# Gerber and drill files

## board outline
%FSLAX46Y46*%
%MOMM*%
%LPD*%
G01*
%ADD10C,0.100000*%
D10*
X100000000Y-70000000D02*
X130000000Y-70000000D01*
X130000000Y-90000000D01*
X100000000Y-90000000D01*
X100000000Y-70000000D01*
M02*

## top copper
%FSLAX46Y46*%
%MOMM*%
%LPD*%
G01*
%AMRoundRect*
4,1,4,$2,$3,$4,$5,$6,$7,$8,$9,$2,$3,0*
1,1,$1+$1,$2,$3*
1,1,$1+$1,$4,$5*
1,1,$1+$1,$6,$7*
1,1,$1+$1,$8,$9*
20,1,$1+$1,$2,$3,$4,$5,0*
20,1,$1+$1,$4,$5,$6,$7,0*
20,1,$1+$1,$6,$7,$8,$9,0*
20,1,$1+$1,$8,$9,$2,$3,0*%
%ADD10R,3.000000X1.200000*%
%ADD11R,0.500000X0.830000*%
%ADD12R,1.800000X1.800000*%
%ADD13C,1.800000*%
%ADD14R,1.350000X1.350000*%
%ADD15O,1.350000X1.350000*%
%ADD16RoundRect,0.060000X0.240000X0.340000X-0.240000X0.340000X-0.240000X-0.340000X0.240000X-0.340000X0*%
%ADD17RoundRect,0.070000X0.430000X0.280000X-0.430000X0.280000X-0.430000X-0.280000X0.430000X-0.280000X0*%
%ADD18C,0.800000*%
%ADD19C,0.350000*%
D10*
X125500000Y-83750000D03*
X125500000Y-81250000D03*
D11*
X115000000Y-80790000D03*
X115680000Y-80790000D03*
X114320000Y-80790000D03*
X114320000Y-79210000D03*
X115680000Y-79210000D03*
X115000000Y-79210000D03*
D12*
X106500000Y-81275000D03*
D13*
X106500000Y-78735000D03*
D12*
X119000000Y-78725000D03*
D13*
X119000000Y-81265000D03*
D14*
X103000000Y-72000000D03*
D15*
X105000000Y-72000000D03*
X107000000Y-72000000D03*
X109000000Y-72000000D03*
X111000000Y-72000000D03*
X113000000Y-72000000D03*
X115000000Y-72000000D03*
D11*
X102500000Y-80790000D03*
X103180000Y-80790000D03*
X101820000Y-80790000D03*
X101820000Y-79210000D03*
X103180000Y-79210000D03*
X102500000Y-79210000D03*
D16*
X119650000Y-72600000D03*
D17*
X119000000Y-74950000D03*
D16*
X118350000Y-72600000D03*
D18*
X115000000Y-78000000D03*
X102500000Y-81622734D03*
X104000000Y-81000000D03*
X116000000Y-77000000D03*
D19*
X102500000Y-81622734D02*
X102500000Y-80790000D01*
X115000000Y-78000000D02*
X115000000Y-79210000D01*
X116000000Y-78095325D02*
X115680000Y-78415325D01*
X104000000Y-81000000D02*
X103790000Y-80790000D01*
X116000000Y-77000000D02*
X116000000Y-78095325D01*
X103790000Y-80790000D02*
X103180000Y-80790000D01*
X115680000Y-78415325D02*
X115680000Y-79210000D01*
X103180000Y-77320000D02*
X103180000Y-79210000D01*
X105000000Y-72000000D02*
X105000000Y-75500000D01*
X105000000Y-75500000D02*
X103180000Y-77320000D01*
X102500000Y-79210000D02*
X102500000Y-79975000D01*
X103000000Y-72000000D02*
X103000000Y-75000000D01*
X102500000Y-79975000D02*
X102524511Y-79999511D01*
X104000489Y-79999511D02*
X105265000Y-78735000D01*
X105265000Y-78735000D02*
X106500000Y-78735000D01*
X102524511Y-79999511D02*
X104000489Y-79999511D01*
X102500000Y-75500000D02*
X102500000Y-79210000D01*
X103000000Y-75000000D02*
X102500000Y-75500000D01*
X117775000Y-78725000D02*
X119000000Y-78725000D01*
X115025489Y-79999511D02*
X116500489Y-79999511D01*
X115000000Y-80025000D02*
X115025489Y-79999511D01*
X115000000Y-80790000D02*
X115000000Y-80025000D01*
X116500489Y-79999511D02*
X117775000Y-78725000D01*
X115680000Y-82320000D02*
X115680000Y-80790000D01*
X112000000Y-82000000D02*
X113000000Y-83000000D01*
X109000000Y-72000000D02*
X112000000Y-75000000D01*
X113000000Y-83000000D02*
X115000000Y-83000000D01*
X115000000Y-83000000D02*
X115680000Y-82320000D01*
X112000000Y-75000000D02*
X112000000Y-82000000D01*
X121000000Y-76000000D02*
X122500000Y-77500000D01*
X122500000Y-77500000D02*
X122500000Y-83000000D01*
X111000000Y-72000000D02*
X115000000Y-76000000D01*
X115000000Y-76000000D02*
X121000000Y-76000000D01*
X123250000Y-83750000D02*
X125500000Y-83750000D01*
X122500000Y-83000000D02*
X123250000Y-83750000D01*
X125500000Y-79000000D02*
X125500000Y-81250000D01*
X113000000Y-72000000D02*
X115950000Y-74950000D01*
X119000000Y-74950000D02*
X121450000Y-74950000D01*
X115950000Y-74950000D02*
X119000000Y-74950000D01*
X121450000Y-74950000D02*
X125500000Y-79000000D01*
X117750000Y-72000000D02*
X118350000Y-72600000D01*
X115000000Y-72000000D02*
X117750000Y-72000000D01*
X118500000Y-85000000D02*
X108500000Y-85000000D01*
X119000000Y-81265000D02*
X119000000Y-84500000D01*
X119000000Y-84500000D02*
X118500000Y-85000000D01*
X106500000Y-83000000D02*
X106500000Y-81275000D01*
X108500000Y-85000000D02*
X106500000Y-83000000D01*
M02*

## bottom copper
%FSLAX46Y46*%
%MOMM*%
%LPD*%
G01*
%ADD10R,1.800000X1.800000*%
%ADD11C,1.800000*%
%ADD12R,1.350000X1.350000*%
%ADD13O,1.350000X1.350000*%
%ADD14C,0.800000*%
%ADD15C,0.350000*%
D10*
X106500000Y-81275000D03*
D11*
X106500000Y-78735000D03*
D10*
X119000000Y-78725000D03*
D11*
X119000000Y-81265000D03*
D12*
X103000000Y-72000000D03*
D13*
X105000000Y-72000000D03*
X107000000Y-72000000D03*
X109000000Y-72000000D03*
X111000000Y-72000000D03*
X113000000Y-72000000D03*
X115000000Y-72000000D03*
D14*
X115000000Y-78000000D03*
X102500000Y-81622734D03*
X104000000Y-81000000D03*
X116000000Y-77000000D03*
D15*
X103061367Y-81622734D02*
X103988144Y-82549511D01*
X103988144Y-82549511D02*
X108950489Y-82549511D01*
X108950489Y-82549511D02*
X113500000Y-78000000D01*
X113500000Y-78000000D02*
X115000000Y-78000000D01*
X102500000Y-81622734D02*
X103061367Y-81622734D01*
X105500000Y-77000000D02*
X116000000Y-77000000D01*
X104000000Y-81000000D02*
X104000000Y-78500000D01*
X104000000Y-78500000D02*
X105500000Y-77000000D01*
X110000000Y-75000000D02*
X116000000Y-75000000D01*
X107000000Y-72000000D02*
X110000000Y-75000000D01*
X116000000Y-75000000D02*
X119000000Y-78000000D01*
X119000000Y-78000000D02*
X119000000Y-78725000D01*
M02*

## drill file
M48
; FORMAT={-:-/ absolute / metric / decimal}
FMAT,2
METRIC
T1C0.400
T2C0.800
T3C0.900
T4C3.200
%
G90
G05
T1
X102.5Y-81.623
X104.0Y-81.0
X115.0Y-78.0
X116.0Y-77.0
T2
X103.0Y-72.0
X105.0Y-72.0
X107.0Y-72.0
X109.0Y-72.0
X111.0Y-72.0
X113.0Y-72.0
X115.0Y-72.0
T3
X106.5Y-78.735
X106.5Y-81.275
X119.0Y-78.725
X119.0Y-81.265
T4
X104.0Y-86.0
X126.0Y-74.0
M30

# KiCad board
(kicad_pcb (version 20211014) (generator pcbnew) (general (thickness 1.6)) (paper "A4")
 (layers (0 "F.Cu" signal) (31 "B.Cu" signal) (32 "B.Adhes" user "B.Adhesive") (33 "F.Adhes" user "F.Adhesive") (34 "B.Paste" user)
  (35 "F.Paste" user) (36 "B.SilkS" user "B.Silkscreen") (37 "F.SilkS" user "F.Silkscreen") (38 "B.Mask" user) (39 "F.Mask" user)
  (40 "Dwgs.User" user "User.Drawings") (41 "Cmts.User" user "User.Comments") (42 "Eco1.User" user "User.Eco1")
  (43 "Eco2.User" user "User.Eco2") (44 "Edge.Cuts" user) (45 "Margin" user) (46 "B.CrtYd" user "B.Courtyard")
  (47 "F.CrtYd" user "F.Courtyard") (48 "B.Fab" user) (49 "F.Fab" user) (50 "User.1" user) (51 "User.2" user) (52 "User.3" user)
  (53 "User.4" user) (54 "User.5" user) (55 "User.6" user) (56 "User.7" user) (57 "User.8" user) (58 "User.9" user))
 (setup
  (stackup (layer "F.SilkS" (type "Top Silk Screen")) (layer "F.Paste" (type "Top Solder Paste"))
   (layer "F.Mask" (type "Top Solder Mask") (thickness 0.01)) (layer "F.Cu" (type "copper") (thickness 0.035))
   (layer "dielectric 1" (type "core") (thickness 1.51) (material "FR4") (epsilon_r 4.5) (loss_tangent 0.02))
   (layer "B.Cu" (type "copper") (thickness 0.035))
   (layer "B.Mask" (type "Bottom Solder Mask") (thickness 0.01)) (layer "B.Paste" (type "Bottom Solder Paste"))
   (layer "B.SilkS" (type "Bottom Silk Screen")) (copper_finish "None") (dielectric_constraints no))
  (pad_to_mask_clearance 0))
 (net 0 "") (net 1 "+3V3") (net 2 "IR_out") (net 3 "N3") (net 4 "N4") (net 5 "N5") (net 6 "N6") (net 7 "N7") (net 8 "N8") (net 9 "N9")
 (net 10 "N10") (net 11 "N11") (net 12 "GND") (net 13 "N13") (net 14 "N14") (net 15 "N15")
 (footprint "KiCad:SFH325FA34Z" (layer "F.Cu") (at 125.5 82.5 90)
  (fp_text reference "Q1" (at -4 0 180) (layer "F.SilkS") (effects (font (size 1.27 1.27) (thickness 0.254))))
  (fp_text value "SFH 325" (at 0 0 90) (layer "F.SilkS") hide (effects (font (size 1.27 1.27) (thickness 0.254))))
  (pad "1" smd rect (at -1.25 0 90) (size 1.2 3) (layers "F.Cu" "F.Paste" "F.Mask") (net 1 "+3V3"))
  (pad "2" smd rect (at 1.25 0 90) (size 1.2 3) (layers "F.Cu" "F.Paste" "F.Mask") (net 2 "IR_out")))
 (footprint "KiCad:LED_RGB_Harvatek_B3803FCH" (layer "F.Cu") (at 115 80 180)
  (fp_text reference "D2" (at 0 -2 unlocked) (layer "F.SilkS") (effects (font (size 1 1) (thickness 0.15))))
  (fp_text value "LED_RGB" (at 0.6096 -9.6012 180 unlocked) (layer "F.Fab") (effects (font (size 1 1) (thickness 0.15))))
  (pad "1" smd rect (at 0 -0.79 180) (size 0.5 0.83) (layers "F.Cu" "F.Paste" "F.Mask") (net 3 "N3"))
  (pad "2" smd rect (at -0.68 -0.79 180) (size 0.5 0.83) (layers "F.Cu" "F.Paste" "F.Mask") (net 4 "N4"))
  (pad "3" smd rect (at 0.68 -0.79 180) (size 0.5 0.83) (layers "F.Cu" "F.Paste" "F.Mask") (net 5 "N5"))
  (pad "4" smd rect (at 0.68 0.79 180) (size 0.5 0.83) (layers "F.Cu" "F.Paste" "F.Mask") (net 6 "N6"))
  (pad "5" smd rect (at -0.68 0.79 180) (size 0.5 0.83) (layers "F.Cu" "F.Paste" "F.Mask") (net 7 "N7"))
  (pad "6" smd rect (at 0 0.79 180) (size 0.5 0.83) (layers "F.Cu" "F.Paste" "F.Mask") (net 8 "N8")))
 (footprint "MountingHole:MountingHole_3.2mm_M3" (layer "F.Cu") (at 104 86)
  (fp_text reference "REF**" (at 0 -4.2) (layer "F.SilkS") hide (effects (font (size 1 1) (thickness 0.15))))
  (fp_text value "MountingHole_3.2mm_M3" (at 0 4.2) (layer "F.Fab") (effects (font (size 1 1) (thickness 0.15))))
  (pad "" np_thru_hole circle (at 0 0) (size 3.2 3.2) (drill 3.2) (layers *.Cu *.Mask)))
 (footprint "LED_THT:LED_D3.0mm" (layer "F.Cu") (at 106.5 81.275 90)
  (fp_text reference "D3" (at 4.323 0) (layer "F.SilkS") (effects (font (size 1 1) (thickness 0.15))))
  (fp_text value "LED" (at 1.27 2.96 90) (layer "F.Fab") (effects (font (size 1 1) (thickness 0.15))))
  (pad "1" thru_hole rect (at 0 0 90) (size 1.8 1.8) (drill 0.9) (layers *.Cu *.Mask) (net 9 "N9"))
  (pad "2" thru_hole circle (at 2.54 0 90) (size 1.8 1.8) (drill 0.9) (layers *.Cu *.Mask) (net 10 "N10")))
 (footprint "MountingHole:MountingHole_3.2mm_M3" (layer "F.Cu") (at 126 74)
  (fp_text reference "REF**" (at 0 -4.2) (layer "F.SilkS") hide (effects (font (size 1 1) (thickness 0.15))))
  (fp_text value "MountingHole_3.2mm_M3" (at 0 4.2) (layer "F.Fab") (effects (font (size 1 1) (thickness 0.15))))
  (pad "" np_thru_hole circle (at 0 0) (size 3.2 3.2) (drill 3.2) (layers *.Cu *.Mask)))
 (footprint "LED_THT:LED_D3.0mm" (layer "F.Cu") (at 119 78.725 -90)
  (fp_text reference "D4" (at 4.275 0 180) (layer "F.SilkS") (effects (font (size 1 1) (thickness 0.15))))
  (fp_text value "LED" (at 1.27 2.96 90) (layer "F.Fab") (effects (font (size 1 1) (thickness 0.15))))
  (pad "1" thru_hole rect (at 0 0 270) (size 1.8 1.8) (drill 0.9) (layers *.Cu *.Mask) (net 3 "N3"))
  (pad "2" thru_hole circle (at 2.54 0 270) (size 1.8 1.8) (drill 0.9) (layers *.Cu *.Mask) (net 9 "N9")))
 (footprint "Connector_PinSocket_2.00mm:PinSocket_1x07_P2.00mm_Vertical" (layer "F.Cu") (at 103 72 90)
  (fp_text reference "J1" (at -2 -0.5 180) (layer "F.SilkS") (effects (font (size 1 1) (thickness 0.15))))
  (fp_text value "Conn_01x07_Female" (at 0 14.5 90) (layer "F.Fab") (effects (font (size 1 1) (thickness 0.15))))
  (pad "1" thru_hole rect (at 0 0 90) (size 1.35 1.35) (drill 0.8) (layers *.Cu *.Mask) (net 10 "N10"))
  (pad "2" thru_hole oval (at 0 2 90) (size 1.35 1.35) (drill 0.8) (layers *.Cu *.Mask) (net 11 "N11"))
  (pad "3" thru_hole oval (at 0 4 90) (size 1.35 1.35) (drill 0.8) (layers *.Cu *.Mask) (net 3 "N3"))
  (pad "4" thru_hole oval (at 0 6 90) (size 1.35 1.35) (drill 0.8) (layers *.Cu *.Mask) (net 4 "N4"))
  (pad "5" thru_hole oval (at 0 8 90) (size 1.35 1.35) (drill 0.8) (layers *.Cu *.Mask) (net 1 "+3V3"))
  (pad "6" thru_hole oval (at 0 10 90) (size 1.35 1.35) (drill 0.8) (layers *.Cu *.Mask) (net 2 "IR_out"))
  (pad "7" thru_hole oval (at 0 12 90) (size 1.35 1.35) (drill 0.8) (layers *.Cu *.Mask) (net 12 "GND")))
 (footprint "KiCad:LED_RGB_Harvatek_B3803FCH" (layer "F.Cu") (at 102.5 80 180)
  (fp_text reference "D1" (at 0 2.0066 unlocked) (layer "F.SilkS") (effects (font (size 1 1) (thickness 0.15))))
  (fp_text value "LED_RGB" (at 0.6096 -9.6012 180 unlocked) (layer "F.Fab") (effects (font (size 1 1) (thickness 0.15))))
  (pad "1" smd rect (at 0 -0.79 180) (size 0.5 0.83) (layers "F.Cu" "F.Paste" "F.Mask") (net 8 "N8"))
  (pad "2" smd rect (at -0.68 -0.79 180) (size 0.5 0.83) (layers "F.Cu" "F.Paste" "F.Mask") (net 7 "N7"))
  (pad "3" smd rect (at 0.68 -0.79 180) (size 0.5 0.83) (layers "F.Cu" "F.Paste" "F.Mask") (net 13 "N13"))
  (pad "4" smd rect (at 0.68 0.79 180) (size 0.5 0.83) (layers "F.Cu" "F.Paste" "F.Mask") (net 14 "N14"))
  (pad "5" smd rect (at -0.68 0.79 180) (size 0.5 0.83) (layers "F.Cu" "F.Paste" "F.Mask") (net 11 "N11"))
  (pad "6" smd rect (at 0 0.79 180) (size 0.5 0.83) (layers "F.Cu" "F.Paste" "F.Mask") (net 10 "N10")))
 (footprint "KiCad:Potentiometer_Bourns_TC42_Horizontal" (layer "F.Cu") (at 119 74 180)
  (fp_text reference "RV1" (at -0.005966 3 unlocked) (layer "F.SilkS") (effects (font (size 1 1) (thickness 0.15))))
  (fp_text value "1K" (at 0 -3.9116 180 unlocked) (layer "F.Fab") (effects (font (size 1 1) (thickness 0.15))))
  (pad "1" smd roundrect (at -0.65 1.4 180) (size 0.6 0.8) (layers "F.Cu" "F.Paste" "F.Mask") (roundrect_rratio 0.1) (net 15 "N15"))
  (pad "2" smd roundrect (at 0 -0.95 180) (size 1 0.7) (layers "F.Cu" "F.Paste" "F.Mask") (roundrect_rratio 0.1) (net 2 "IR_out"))
  (pad "3" smd roundrect (at 0.65 1.4 180) (size 0.6 0.8) (layers "F.Cu" "F.Paste" "F.Mask") (roundrect_rratio 0.1) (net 12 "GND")))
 (gr_rect (start 100 70) (end 130 90) (layer "Edge.Cuts") (width 0.1) (fill none))
 (segment (start 102.5 81.622734) (end 102.5 80.79) (width 0.35) (layer "F.Cu") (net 8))
 (segment (start 115 78) (end 115 79.21) (width 0.35) (layer "F.Cu") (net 8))
 (via (at 115 78) (size 0.8) (drill 0.4) (layers "F.Cu" "B.Cu") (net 8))
 (via (at 102.5 81.622734) (size 0.8) (drill 0.4) (layers "F.Cu" "B.Cu") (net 8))
 (segment (start 103.061367 81.622734) (end 103.988144 82.549511) (width 0.35) (layer "B.Cu") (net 8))
 (segment (start 103.988144 82.549511) (end 108.950489 82.549511) (width 0.35) (layer "B.Cu") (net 8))
 (segment (start 108.950489 82.549511) (end 113.5 78) (width 0.35) (layer "B.Cu") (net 8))
 (segment (start 113.5 78) (end 115 78) (width 0.35) (layer "B.Cu") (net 8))
 (segment (start 102.5 81.622734) (end 103.061367 81.622734) (width 0.35) (layer "B.Cu") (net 8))
 (segment (start 116 78.095325) (end 115.68 78.415325) (width 0.35) (layer "F.Cu") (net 7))
 (segment (start 104 81) (end 103.79 80.79) (width 0.35) (layer "F.Cu") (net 7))
 (segment (start 116 77) (end 116 78.095325) (width 0.35) (layer "F.Cu") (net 7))
 (segment (start 103.79 80.79) (end 103.18 80.79) (width 0.35) (layer "F.Cu") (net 7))
 (segment (start 115.68 78.415325) (end 115.68 79.21) (width 0.35) (layer "F.Cu") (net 7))
 (via (at 104 81) (size 0.8) (drill 0.4) (layers "F.Cu" "B.Cu") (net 7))
 (via (at 116 77) (size 0.8) (drill 0.4) (layers "F.Cu" "B.Cu") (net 7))
 (segment (start 105.5 77) (end 116 77) (width 0.35) (layer "B.Cu") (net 7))
 (segment (start 104 81) (end 104 78.5) (width 0.35) (layer "B.Cu") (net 7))
 (segment (start 104 78.5) (end 105.5 77) (width 0.35) (layer "B.Cu") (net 7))
 (segment (start 103.18 77.32) (end 103.18 79.21) (width 0.35) (layer "F.Cu") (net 11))
 (segment (start 105 72) (end 105 75.5) (width 0.35) (layer "F.Cu") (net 11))
 (segment (start 105 75.5) (end 103.18 77.32) (width 0.35) (layer "F.Cu") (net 11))
 (segment (start 102.5 79.21) (end 102.5 79.975) (width 0.35) (layer "F.Cu") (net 10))
 (segment (start 103 72) (end 103 75) (width 0.35) (layer "F.Cu") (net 10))
 (segment (start 102.5 79.975) (end 102.524511 79.999511) (width 0.35) (layer "F.Cu") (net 10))
 (segment (start 104.000489 79.999511) (end 105.265 78.735) (width 0.35) (layer "F.Cu") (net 10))
 (segment (start 105.265 78.735) (end 106.5 78.735) (width 0.35) (layer "F.Cu") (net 10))
 (segment (start 102.524511 79.999511) (end 104.000489 79.999511) (width 0.35) (layer "F.Cu") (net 10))
 (segment (start 102.5 75.5) (end 102.5 79.21) (width 0.35) (layer "F.Cu") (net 10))
 (segment (start 103 75) (end 102.5 75.5) (width 0.35) (layer "F.Cu") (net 10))
 (segment (start 117.775 78.725) (end 119 78.725) (width 0.35) (layer "F.Cu") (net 3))
 (segment (start 115.025489 79.999511) (end 116.500489 79.999511) (width 0.35) (layer "F.Cu") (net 3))
 (segment (start 115 80.025) (end 115.025489 79.999511) (width 0.35) (layer "F.Cu") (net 3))
 (segment (start 115 80.79) (end 115 80.025) (width 0.35) (layer "F.Cu") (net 3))
 (segment (start 116.500489 79.999511) (end 117.775 78.725) (width 0.35) (layer "F.Cu") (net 3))
 (segment (start 110 75) (end 116 75) (width 0.35) (layer "B.Cu") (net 3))
 (segment (start 107 72) (end 110 75) (width 0.35) (layer "B.Cu") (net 3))
 (segment (start 116 75) (end 119 78) (width 0.35) (layer "B.Cu") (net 3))
 (segment (start 119 78) (end 119 78.725) (width 0.35) (layer "B.Cu") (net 3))
 (segment (start 115.68 82.32) (end 115.68 80.79) (width 0.35) (layer "F.Cu") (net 4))
 (segment (start 112 82) (end 113 83) (width 0.35) (layer "F.Cu") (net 4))
 (segment (start 109 72) (end 112 75) (width 0.35) (layer "F.Cu") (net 4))
 (segment (start 113 83) (end 115 83) (width 0.35) (layer "F.Cu") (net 4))
 (segment (start 115 83) (end 115.68 82.32) (width 0.35) (layer "F.Cu") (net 4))
 (segment (start 112 75) (end 112 82) (width 0.35) (layer "F.Cu") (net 4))
 (segment (start 121 76) (end 122.5 77.5) (width 0.35) (layer "F.Cu") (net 1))
 (segment (start 122.5 77.5) (end 122.5 83) (width 0.35) (layer "F.Cu") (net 1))
 (segment (start 111 72) (end 115 76) (width 0.35) (layer "F.Cu") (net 1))
 (segment (start 115 76) (end 121 76) (width 0.35) (layer "F.Cu") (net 1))
 (segment (start 123.25 83.75) (end 125.5 83.75) (width 0.35) (layer "F.Cu") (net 1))
 (segment (start 122.5 83) (end 123.25 83.75) (width 0.35) (layer "F.Cu") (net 1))
 (segment (start 125.5 79) (end 125.5 81.25) (width 0.35) (layer "F.Cu") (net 2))
 (segment (start 113 72) (end 115.95 74.95) (width 0.35) (layer "F.Cu") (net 2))
 (segment (start 119 74.95) (end 121.45 74.95) (width 0.35) (layer "F.Cu") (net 2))
 (segment (start 115.95 74.95) (end 119 74.95) (width 0.35) (layer "F.Cu") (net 2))
 (segment (start 121.45 74.95) (end 125.5 79) (width 0.35) (layer "F.Cu") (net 2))
 (segment (start 117.75 72) (end 118.35 72.6) (width 0.35) (layer "F.Cu") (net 12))
 (segment (start 115 72) (end 117.75 72) (width 0.35) (layer "F.Cu") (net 12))
 (segment (start 118.5 85) (end 108.5 85) (width 0.35) (layer "F.Cu") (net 9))
 (segment (start 119 81.265) (end 119 84.5) (width 0.35) (layer "F.Cu") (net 9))
 (segment (start 119 84.5) (end 118.5 85) (width 0.35) (layer "F.Cu") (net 9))
 (segment (start 106.5 83) (end 106.5 81.275) (width 0.35) (layer "F.Cu") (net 9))
 (segment (start 108.5 85) (end 106.5 83) (width 0.35) (layer "F.Cu") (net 9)))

